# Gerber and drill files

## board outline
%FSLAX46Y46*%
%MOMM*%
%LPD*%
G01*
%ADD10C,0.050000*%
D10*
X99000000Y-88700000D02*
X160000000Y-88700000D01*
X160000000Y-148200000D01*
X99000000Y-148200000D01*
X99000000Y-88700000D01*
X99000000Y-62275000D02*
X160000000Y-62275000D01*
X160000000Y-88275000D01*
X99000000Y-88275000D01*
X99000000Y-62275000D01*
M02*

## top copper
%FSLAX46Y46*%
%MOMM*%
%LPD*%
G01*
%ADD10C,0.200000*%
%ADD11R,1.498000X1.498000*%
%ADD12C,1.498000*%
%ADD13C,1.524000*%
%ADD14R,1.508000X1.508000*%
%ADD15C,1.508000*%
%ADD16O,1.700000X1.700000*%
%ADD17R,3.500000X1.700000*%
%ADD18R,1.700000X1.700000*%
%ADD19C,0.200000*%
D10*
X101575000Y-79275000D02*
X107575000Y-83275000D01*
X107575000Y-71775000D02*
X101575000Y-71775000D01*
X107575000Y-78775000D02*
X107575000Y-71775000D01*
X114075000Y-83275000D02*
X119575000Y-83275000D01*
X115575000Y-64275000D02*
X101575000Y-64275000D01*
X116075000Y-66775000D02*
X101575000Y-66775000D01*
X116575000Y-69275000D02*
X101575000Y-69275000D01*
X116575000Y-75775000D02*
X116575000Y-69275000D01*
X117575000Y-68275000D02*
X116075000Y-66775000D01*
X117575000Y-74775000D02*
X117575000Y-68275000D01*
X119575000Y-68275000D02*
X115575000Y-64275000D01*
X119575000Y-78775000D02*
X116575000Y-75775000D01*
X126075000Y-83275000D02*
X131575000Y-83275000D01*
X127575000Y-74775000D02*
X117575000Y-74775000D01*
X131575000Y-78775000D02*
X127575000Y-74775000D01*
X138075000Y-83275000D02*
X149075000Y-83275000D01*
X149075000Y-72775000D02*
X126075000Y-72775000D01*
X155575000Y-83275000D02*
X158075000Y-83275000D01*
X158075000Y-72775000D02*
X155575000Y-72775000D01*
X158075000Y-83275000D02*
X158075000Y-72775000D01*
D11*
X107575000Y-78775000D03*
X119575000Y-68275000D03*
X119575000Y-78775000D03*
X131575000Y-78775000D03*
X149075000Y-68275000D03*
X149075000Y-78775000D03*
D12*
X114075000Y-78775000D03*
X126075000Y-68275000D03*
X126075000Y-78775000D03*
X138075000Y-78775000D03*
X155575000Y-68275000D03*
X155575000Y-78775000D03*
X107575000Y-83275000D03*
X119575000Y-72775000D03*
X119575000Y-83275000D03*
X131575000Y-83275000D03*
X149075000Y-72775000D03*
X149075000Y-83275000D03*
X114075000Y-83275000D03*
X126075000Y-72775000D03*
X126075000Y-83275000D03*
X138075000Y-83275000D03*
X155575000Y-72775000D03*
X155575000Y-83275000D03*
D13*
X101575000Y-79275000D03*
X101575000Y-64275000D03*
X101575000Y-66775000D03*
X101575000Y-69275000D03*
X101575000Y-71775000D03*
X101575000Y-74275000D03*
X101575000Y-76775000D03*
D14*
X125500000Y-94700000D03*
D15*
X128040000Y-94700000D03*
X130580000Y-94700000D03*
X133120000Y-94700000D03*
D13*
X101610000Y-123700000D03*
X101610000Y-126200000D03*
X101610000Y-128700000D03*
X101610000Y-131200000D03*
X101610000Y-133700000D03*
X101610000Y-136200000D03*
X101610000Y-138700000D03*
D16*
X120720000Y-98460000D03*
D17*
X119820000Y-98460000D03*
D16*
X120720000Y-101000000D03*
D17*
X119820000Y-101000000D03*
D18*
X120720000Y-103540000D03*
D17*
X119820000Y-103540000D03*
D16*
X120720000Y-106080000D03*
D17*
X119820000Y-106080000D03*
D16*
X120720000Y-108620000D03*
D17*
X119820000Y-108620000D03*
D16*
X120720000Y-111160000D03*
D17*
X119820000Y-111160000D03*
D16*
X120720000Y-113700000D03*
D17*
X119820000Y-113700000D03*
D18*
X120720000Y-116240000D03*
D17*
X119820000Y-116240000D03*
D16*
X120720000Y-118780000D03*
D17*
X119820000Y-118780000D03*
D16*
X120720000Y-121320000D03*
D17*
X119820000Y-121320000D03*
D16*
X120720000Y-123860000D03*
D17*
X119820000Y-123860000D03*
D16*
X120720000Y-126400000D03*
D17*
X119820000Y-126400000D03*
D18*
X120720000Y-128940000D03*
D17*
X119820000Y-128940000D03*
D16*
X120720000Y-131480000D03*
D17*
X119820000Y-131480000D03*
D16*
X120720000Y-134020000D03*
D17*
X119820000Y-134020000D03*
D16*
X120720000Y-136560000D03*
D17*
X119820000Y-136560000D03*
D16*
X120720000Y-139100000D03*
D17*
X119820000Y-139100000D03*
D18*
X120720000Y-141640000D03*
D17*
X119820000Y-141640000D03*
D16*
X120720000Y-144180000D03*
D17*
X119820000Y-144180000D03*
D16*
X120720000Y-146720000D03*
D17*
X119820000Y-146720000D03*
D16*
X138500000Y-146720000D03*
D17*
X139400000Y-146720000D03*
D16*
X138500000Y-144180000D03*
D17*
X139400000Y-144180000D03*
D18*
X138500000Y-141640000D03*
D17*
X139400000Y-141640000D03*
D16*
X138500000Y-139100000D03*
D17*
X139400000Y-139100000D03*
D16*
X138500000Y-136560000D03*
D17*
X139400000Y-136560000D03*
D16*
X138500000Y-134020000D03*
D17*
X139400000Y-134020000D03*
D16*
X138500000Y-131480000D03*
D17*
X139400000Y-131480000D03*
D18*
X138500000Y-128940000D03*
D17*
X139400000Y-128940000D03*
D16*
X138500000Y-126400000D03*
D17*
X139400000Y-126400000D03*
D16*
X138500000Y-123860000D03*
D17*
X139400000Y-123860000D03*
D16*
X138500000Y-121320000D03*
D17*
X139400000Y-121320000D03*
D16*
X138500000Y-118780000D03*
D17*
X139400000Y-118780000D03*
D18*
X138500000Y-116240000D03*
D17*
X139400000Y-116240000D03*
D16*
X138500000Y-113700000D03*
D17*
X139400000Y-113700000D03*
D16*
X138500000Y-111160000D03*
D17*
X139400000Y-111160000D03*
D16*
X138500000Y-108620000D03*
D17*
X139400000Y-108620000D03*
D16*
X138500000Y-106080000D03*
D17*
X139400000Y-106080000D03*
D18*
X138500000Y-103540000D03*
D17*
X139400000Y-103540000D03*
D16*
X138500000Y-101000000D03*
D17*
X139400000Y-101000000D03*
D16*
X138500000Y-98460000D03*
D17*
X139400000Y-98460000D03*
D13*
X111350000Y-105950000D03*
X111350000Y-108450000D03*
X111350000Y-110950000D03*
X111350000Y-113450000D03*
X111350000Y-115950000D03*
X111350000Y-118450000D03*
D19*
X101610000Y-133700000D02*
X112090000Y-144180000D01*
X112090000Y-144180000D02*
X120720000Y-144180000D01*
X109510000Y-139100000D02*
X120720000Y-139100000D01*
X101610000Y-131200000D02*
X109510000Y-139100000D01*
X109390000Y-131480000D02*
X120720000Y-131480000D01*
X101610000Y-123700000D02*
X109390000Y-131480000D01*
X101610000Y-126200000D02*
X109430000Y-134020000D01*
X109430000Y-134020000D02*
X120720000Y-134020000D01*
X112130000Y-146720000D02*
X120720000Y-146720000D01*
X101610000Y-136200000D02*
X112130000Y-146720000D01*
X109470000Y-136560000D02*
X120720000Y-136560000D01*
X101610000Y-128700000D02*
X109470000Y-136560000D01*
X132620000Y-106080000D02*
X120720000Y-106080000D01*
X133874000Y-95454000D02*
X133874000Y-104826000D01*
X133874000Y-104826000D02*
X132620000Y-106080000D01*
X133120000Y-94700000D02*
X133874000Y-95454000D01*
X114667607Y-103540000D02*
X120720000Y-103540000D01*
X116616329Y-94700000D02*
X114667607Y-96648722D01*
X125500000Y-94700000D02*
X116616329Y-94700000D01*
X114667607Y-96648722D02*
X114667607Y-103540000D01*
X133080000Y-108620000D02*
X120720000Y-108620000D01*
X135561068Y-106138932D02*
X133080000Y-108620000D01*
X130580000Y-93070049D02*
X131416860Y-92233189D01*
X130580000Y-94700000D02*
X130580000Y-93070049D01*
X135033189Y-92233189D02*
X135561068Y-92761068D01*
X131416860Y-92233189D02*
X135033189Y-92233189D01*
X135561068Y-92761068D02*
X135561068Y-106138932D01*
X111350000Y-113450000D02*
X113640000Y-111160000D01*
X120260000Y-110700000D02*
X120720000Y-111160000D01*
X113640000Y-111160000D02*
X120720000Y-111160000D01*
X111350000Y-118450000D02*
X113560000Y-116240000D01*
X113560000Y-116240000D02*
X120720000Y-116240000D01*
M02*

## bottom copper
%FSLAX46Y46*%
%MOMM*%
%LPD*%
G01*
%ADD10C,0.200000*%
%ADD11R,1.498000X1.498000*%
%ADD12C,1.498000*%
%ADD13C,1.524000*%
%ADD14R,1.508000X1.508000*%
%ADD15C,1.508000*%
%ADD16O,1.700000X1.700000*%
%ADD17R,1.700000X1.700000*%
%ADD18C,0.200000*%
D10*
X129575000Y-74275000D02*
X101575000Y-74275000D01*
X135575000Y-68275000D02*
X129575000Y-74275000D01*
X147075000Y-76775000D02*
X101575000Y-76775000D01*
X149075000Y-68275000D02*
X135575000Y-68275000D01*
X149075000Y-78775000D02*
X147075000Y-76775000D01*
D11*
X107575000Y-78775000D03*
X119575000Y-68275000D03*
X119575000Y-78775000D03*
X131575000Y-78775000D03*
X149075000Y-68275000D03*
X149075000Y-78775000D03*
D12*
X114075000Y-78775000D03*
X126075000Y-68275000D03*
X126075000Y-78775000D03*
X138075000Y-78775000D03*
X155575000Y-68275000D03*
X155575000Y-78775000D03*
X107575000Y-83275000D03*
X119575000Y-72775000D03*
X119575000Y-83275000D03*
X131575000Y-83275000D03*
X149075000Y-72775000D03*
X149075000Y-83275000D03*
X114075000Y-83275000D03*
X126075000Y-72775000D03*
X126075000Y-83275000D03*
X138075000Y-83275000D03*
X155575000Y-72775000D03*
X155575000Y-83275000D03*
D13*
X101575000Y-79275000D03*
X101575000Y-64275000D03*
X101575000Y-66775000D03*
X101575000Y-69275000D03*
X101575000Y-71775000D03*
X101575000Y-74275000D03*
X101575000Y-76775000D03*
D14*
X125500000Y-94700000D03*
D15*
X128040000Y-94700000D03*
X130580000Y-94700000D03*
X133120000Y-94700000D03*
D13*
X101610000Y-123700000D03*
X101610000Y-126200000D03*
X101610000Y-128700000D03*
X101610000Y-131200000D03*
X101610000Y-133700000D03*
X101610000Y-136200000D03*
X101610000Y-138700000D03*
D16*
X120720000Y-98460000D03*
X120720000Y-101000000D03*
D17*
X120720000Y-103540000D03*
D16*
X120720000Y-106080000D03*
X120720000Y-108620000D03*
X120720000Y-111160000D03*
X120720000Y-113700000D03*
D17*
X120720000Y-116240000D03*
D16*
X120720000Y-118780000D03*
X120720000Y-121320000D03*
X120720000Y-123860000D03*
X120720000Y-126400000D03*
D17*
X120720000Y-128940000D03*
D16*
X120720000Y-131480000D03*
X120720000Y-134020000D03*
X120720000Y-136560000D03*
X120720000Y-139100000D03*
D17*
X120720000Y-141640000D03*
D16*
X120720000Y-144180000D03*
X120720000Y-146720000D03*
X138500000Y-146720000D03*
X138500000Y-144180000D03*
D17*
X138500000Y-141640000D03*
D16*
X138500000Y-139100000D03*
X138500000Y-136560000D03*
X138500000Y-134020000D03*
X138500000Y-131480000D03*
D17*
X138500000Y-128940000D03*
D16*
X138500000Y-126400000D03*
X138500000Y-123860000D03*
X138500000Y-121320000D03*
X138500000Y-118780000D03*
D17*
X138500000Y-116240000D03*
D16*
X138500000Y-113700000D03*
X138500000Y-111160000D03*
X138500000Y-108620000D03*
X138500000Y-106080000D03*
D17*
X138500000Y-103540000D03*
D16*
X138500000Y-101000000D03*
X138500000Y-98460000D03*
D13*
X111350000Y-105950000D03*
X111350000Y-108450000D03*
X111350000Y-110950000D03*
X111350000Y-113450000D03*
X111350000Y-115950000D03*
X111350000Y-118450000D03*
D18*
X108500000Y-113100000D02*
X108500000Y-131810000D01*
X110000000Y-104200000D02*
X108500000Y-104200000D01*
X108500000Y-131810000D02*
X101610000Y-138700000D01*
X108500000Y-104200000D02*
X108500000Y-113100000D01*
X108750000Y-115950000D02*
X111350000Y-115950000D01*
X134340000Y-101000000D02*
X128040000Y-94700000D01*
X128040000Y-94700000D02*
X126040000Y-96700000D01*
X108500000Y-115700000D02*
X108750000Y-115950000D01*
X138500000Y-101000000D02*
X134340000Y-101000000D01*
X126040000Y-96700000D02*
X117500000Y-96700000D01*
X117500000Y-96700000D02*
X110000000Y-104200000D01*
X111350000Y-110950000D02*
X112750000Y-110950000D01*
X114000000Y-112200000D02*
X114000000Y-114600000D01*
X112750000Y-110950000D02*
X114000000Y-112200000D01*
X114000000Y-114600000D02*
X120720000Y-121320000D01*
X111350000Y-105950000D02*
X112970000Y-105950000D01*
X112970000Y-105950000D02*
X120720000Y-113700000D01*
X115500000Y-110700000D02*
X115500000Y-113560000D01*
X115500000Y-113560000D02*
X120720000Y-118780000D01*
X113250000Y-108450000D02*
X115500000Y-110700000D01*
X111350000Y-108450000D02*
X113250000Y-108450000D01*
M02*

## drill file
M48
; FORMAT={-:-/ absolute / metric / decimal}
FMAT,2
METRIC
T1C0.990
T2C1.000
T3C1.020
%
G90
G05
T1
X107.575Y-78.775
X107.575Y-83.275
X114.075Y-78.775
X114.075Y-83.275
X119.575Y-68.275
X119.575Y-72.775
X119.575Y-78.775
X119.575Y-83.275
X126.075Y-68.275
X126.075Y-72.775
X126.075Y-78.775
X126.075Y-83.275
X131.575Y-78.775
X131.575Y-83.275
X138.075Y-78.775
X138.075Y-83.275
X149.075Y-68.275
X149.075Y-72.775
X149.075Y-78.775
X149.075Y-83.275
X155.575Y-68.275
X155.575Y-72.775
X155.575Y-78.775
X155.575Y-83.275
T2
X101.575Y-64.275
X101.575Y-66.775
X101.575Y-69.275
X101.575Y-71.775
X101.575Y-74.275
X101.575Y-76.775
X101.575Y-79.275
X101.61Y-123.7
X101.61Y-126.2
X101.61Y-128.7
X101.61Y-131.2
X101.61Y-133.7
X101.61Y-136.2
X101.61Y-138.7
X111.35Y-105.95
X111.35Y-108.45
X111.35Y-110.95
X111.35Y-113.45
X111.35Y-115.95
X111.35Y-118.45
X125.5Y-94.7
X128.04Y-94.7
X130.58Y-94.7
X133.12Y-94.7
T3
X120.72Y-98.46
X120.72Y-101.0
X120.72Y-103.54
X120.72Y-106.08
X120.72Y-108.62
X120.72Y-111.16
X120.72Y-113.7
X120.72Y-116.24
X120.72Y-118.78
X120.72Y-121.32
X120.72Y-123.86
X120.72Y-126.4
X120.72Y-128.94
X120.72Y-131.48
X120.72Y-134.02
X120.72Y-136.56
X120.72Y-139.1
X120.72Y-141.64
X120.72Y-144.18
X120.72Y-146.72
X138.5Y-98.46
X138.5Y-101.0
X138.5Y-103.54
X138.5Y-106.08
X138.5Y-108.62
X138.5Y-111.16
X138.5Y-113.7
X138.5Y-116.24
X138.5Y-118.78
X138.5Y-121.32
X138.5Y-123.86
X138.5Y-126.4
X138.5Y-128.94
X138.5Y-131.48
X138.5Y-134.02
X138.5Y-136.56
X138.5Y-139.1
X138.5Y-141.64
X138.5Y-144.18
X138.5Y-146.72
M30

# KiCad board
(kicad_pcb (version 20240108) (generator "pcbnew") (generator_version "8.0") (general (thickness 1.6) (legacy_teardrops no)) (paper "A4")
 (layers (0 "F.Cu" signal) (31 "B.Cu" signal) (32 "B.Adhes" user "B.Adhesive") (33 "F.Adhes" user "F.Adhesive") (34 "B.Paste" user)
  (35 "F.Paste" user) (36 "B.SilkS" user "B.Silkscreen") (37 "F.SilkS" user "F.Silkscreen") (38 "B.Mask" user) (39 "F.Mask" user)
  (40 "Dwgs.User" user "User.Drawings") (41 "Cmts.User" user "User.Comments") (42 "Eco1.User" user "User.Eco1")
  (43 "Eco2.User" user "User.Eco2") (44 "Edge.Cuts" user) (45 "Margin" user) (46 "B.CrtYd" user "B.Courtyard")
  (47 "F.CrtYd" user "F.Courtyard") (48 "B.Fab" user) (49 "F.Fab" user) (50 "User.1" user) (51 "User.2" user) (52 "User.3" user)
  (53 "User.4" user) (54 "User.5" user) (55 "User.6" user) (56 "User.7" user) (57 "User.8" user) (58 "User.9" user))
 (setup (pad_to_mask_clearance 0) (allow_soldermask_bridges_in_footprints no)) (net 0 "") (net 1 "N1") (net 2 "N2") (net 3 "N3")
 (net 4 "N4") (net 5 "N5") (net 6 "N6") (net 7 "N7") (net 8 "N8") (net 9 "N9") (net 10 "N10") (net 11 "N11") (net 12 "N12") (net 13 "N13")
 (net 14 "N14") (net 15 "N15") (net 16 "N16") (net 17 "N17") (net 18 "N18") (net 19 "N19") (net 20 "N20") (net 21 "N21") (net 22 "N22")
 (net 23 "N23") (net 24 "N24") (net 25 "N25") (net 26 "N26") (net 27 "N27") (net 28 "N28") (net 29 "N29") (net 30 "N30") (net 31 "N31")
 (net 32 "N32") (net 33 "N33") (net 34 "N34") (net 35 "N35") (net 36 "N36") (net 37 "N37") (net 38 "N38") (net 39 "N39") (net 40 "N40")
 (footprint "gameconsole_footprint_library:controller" (layer "F.Cu") (at 99.575 62.775)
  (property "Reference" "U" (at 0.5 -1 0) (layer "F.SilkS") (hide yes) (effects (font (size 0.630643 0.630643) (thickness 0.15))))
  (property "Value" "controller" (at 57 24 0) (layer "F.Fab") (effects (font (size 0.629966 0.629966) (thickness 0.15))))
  (fp_line (start 2 16.5) (end 8 20.5) (stroke (width 0.2) (type default)) (layer "F.Cu"))
  (fp_line (start 8 9) (end 2 9) (stroke (width 0.2) (type default)) (layer "F.Cu"))
  (fp_line (start 8 16) (end 8 9) (stroke (width 0.2) (type default)) (layer "F.Cu"))
  (fp_line (start 14.5 20.5) (end 20 20.5) (stroke (width 0.2) (type default)) (layer "F.Cu"))
  (fp_line (start 16 1.5) (end 2 1.5) (stroke (width 0.2) (type default)) (layer "F.Cu"))
  (fp_line (start 16.5 4) (end 2 4) (stroke (width 0.2) (type default)) (layer "F.Cu"))
  (fp_line (start 17 6.5) (end 2 6.5) (stroke (width 0.2) (type default)) (layer "F.Cu"))
  (fp_line (start 17 13) (end 17 6.5) (stroke (width 0.2) (type default)) (layer "F.Cu"))
  (fp_line (start 18 5.5) (end 16.5 4) (stroke (width 0.2) (type default)) (layer "F.Cu"))
  (fp_line (start 18 12) (end 18 5.5) (stroke (width 0.2) (type default)) (layer "F.Cu"))
  (fp_line (start 20 5.5) (end 16 1.5) (stroke (width 0.2) (type default)) (layer "F.Cu"))
  (fp_line (start 20 16) (end 17 13) (stroke (width 0.2) (type default)) (layer "F.Cu"))
  (fp_line (start 26.5 20.5) (end 32 20.5) (stroke (width 0.2) (type default)) (layer "F.Cu"))
  (fp_line (start 28 12) (end 18 12) (stroke (width 0.2) (type default)) (layer "F.Cu"))
  (fp_line (start 32 16) (end 28 12) (stroke (width 0.2) (type default)) (layer "F.Cu"))
  (fp_line (start 38.5 20.5) (end 49.5 20.5) (stroke (width 0.2) (type default)) (layer "F.Cu"))
  (fp_line (start 49.5 10) (end 26.5 10) (stroke (width 0.2) (type default)) (layer "F.Cu"))
  (fp_line (start 56 20.5) (end 58.5 20.5) (stroke (width 0.2) (type default)) (layer "F.Cu"))
  (fp_line (start 58.5 10) (end 56 10) (stroke (width 0.2) (type default)) (layer "F.Cu"))
  (fp_line (start 58.5 20.5) (end 58.5 10) (stroke (width 0.2) (type default)) (layer "F.Cu"))
  (fp_line (start 30 11.5) (end 2 11.5) (stroke (width 0.2) (type default)) (layer "B.Cu"))
  (fp_line (start 36 5.5) (end 30 11.5) (stroke (width 0.2) (type default)) (layer "B.Cu"))
  (fp_line (start 47.5 14) (end 2 14) (stroke (width 0.2) (type default)) (layer "B.Cu"))
  (fp_line (start 49.5 5.5) (end 36 5.5) (stroke (width 0.2) (type default)) (layer "B.Cu"))
  (fp_line (start 49.5 16) (end 47.5 14) (stroke (width 0.2) (type default)) (layer "B.Cu"))
  (pad "1" thru_hole rect (at 8 16) (size 1.498 1.498) (drill 0.99) (layers "*.Cu" "*.Mask") (remove_unused_layers no)
   (solder_mask_margin 0.102))
  (pad "1" thru_hole rect (at 20 5.5) (size 1.498 1.498) (drill 0.99) (layers "*.Cu" "*.Mask") (remove_unused_layers no)
   (solder_mask_margin 0.102))
  (pad "1" thru_hole rect (at 20 16) (size 1.498 1.498) (drill 0.99) (layers "*.Cu" "*.Mask") (remove_unused_layers no)
   (solder_mask_margin 0.102))
  (pad "1" thru_hole rect (at 32 16) (size 1.498 1.498) (drill 0.99) (layers "*.Cu" "*.Mask") (remove_unused_layers no)
   (solder_mask_margin 0.102))
  (pad "1" thru_hole rect (at 49.5 5.5) (size 1.498 1.498) (drill 0.99) (layers "*.Cu" "*.Mask") (remove_unused_layers no)
   (solder_mask_margin 0.102))
  (pad "1" thru_hole rect (at 49.5 16) (size 1.498 1.498) (drill 0.99) (layers "*.Cu" "*.Mask") (remove_unused_layers no)
   (solder_mask_margin 0.102))
  (pad "2" thru_hole circle (at 14.5 16) (size 1.498 1.498) (drill 0.99) (layers "*.Cu" "*.Mask") (remove_unused_layers no)
   (solder_mask_margin 0.102))
  (pad "2" thru_hole circle (at 26.5 5.5) (size 1.498 1.498) (drill 0.99) (layers "*.Cu" "*.Mask") (remove_unused_layers no)
   (solder_mask_margin 0.102))
  (pad "2" thru_hole circle (at 26.5 16) (size 1.498 1.498) (drill 0.99) (layers "*.Cu" "*.Mask") (remove_unused_layers no)
   (solder_mask_margin 0.102))
  (pad "2" thru_hole circle (at 38.5 16) (size 1.498 1.498) (drill 0.99) (layers "*.Cu" "*.Mask") (remove_unused_layers no)
   (solder_mask_margin 0.102))
  (pad "2" thru_hole circle (at 56 5.5) (size 1.498 1.498) (drill 0.99) (layers "*.Cu" "*.Mask") (remove_unused_layers no)
   (solder_mask_margin 0.102))
  (pad "2" thru_hole circle (at 56 16) (size 1.498 1.498) (drill 0.99) (layers "*.Cu" "*.Mask") (remove_unused_layers no)
   (solder_mask_margin 0.102))
  (pad "3" thru_hole circle (at 8 20.5) (size 1.498 1.498) (drill 0.99) (layers "*.Cu" "*.Mask") (remove_unused_layers no)
   (solder_mask_margin 0.102))
  (pad "3" thru_hole circle (at 20 10) (size 1.498 1.498) (drill 0.99) (layers "*.Cu" "*.Mask") (remove_unused_layers no)
   (solder_mask_margin 0.102))
  (pad "3" thru_hole circle (at 20 20.5) (size 1.498 1.498) (drill 0.99) (layers "*.Cu" "*.Mask") (remove_unused_layers no)
   (solder_mask_margin 0.102))
  (pad "3" thru_hole circle (at 32 20.5) (size 1.498 1.498) (drill 0.99) (layers "*.Cu" "*.Mask") (remove_unused_layers no)
   (solder_mask_margin 0.102))
  (pad "3" thru_hole circle (at 49.5 10) (size 1.498 1.498) (drill 0.99) (layers "*.Cu" "*.Mask") (remove_unused_layers no)
   (solder_mask_margin 0.102))
  (pad "3" thru_hole circle (at 49.5 20.5) (size 1.498 1.498) (drill 0.99) (layers "*.Cu" "*.Mask") (remove_unused_layers no)
   (solder_mask_margin 0.102))
  (pad "4" thru_hole circle (at 14.5 20.5) (size 1.498 1.498) (drill 0.99) (layers "*.Cu" "*.Mask") (remove_unused_layers no)
   (solder_mask_margin 0.102))
  (pad "4" thru_hole circle (at 26.5 10) (size 1.498 1.498) (drill 0.99) (layers "*.Cu" "*.Mask") (remove_unused_layers no)
   (solder_mask_margin 0.102))
  (pad "4" thru_hole circle (at 26.5 20.5) (size 1.498 1.498) (drill 0.99) (layers "*.Cu" "*.Mask") (remove_unused_layers no)
   (solder_mask_margin 0.102))
  (pad "4" thru_hole circle (at 38.5 20.5) (size 1.498 1.498) (drill 0.99) (layers "*.Cu" "*.Mask") (remove_unused_layers no)
   (solder_mask_margin 0.102))
  (pad "4" thru_hole circle (at 56 10) (size 1.498 1.498) (drill 0.99) (layers "*.Cu" "*.Mask") (remove_unused_layers no)
   (solder_mask_margin 0.102))
  (pad "4" thru_hole circle (at 56 20.5) (size 1.498 1.498) (drill 0.99) (layers "*.Cu" "*.Mask") (remove_unused_layers no)
   (solder_mask_margin 0.102))
  (pad "5" thru_hole circle (at 2 16.5) (size 1.524 1.524) (drill 1) (layers "*.Cu" "*.Mask") (remove_unused_layers no))
  (pad "6" thru_hole circle (at 2 1.5) (size 1.524 1.524) (drill 1) (layers "*.Cu" "*.Mask") (remove_unused_layers no))
  (pad "7" thru_hole circle (at 2 4) (size 1.524 1.524) (drill 1) (layers "*.Cu" "*.Mask") (remove_unused_layers no))
  (pad "8" thru_hole circle (at 2 6.5) (size 1.524 1.524) (drill 1) (layers "*.Cu" "*.Mask") (remove_unused_layers no))
  (pad "9" thru_hole circle (at 2 9) (size 1.524 1.524) (drill 1) (layers "*.Cu" "*.Mask") (remove_unused_layers no))
  (pad "10" thru_hole circle (at 2 11.5) (size 1.524 1.524) (drill 1) (layers "*.Cu" "*.Mask") (remove_unused_layers no))
  (pad "11" thru_hole circle (at 2 14) (size 1.524 1.524) (drill 1) (layers "*.Cu" "*.Mask") (remove_unused_layers no)))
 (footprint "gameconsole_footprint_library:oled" (layer "F.Cu") (at 129.31 106.2)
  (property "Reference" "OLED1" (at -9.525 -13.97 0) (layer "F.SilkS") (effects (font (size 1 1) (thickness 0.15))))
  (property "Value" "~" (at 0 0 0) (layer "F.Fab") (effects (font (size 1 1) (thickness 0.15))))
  (pad "1" thru_hole rect (at -3.81 -11.5) (size 1.508 1.508) (drill 1) (layers "*.Cu" "*.Mask") (remove_unused_layers no) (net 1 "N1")
   (solder_mask_margin 0.102))
  (pad "2" thru_hole circle (at -1.27 -11.5) (size 1.508 1.508) (drill 1) (layers "*.Cu" "*.Mask") (remove_unused_layers no) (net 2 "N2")
   (solder_mask_margin 0.102))
  (pad "3" thru_hole circle (at 1.27 -11.5) (size 1.508 1.508) (drill 1) (layers "*.Cu" "*.Mask") (remove_unused_layers no) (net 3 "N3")
   (solder_mask_margin 0.102))
  (pad "4" thru_hole circle (at 3.81 -11.5) (size 1.508 1.508) (drill 1) (layers "*.Cu" "*.Mask") (remove_unused_layers no) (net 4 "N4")
   (solder_mask_margin 0.102)))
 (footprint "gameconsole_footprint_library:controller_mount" (layer "F.Cu") (at 129.61 134.2)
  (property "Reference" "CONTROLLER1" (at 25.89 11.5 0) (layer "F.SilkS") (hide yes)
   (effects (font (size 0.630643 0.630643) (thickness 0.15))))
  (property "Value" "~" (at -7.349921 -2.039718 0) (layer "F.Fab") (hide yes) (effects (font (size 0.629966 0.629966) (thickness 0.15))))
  (pad "1" thru_hole circle (at -28 -10.5) (size 1.524 1.524) (drill 1) (layers "*.Cu" "*.Mask") (remove_unused_layers no) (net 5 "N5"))
  (pad "2" thru_hole circle (at -28 -8) (size 1.524 1.524) (drill 1) (layers "*.Cu" "*.Mask") (remove_unused_layers no) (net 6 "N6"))
  (pad "3" thru_hole circle (at -28 -5.5) (size 1.524 1.524) (drill 1) (layers "*.Cu" "*.Mask") (remove_unused_layers no) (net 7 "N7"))
  (pad "4" thru_hole circle (at -28 -3) (size 1.524 1.524) (drill 1) (layers "*.Cu" "*.Mask") (remove_unused_layers no) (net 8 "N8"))
  (pad "5" thru_hole circle (at -28 -0.5) (size 1.524 1.524) (drill 1) (layers "*.Cu" "*.Mask") (remove_unused_layers no) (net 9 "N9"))
  (pad "6" thru_hole circle (at -28 2) (size 1.524 1.524) (drill 1) (layers "*.Cu" "*.Mask") (remove_unused_layers no) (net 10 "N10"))
  (pad "7" thru_hole circle (at -28 4.5) (size 1.524 1.524) (drill 1) (layers "*.Cu" "*.Mask") (remove_unused_layers no) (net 2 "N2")))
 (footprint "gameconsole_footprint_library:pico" (layer "F.Cu") (at 129.61 122.59)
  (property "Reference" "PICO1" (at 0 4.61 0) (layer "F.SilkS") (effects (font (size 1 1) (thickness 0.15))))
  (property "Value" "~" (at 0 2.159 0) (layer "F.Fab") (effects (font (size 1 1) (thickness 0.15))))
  (pad "1" thru_hole oval (at -8.89 -24.13) (size 1.7 1.7) (drill 1.02) (layers "*.Cu" "*.Mask") (remove_unused_layers no) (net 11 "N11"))
  (pad "1" smd rect (at -8.89 -24.13) (size 3.5 1.7) (drill (offset -0.9 0)) (layers "F.Cu" "F.Mask") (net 11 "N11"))
  (pad "2" thru_hole oval (at -8.89 -21.59) (size 1.7 1.7) (drill 1.02) (layers "*.Cu" "*.Mask") (remove_unused_layers no) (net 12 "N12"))
  (pad "2" smd rect (at -8.89 -21.59) (size 3.5 1.7) (drill (offset -0.9 0)) (layers "F.Cu" "F.Mask") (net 12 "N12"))
  (pad "3" thru_hole rect (at -8.89 -19.05) (size 1.7 1.7) (drill 1.02) (layers "*.Cu" "*.Mask") (remove_unused_layers no) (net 1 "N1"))
  (pad "3" smd rect (at -8.89 -19.05) (size 3.5 1.7) (drill (offset -0.9 0)) (layers "F.Cu" "F.Mask") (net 1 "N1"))
  (pad "4" thru_hole oval (at -8.89 -16.51) (size 1.7 1.7) (drill 1.02) (layers "*.Cu" "*.Mask") (remove_unused_layers no) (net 4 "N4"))
  (pad "4" smd rect (at -8.89 -16.51) (size 3.5 1.7) (drill (offset -0.9 0)) (layers "F.Cu" "F.Mask") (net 4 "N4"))
  (pad "5" thru_hole oval (at -8.89 -13.97) (size 1.7 1.7) (drill 1.02) (layers "*.Cu" "*.Mask") (remove_unused_layers no) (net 3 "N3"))
  (pad "5" smd rect (at -8.89 -13.97) (size 3.5 1.7) (drill (offset -0.9 0)) (layers "F.Cu" "F.Mask") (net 3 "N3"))
  (pad "6" thru_hole oval (at -8.89 -11.43) (size 1.7 1.7) (drill 1.02) (layers "*.Cu" "*.Mask") (remove_unused_layers no) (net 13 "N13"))
  (pad "6" smd rect (at -8.89 -11.43) (size 3.5 1.7) (drill (offset -0.9 0)) (layers "F.Cu" "F.Mask") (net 13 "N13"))
  (pad "7" thru_hole oval (at -8.89 -8.89) (size 1.7 1.7) (drill 1.02) (layers "*.Cu" "*.Mask") (remove_unused_layers no) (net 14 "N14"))
  (pad "7" smd rect (at -8.89 -8.89) (size 3.5 1.7) (drill (offset -0.9 0)) (layers "F.Cu" "F.Mask") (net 14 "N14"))
  (pad "8" thru_hole rect (at -8.89 -6.35) (size 1.7 1.7) (drill 1.02) (layers "*.Cu" "*.Mask") (remove_unused_layers no) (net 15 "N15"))
  (pad "8" smd rect (at -8.89 -6.35) (size 3.5 1.7) (drill (offset -0.9 0)) (layers "F.Cu" "F.Mask") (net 15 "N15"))
  (pad "9" thru_hole oval (at -8.89 -3.81) (size 1.7 1.7) (drill 1.02) (layers "*.Cu" "*.Mask") (remove_unused_layers no) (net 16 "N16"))
  (pad "9" smd rect (at -8.89 -3.81) (size 3.5 1.7) (drill (offset -0.9 0)) (layers "F.Cu" "F.Mask") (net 16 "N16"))
  (pad "10" thru_hole oval (at -8.89 -1.27) (size 1.7 1.7) (drill 1.02) (layers "*.Cu" "*.Mask") (remove_unused_layers no) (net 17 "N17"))
  (pad "10" smd rect (at -8.89 -1.27) (size 3.5 1.7) (drill (offset -0.9 0)) (layers "F.Cu" "F.Mask") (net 17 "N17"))
  (pad "11" thru_hole oval (at -8.89 1.27) (size 1.7 1.7) (drill 1.02) (layers "*.Cu" "*.Mask") (remove_unused_layers no) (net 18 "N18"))
  (pad "11" smd rect (at -8.89 1.27) (size 3.5 1.7) (drill (offset -0.9 0)) (layers "F.Cu" "F.Mask") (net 18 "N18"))
  (pad "12" thru_hole oval (at -8.89 3.81) (size 1.7 1.7) (drill 1.02) (layers "*.Cu" "*.Mask") (remove_unused_layers no) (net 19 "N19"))
  (pad "12" smd rect (at -8.89 3.81) (size 3.5 1.7) (drill (offset -0.9 0)) (layers "F.Cu" "F.Mask") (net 19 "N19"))
  (pad "13" thru_hole rect (at -8.89 6.35) (size 1.7 1.7) (drill 1.02) (layers "*.Cu" "*.Mask") (remove_unused_layers no) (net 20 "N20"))
  (pad "13" smd rect (at -8.89 6.35) (size 3.5 1.7) (drill (offset -0.9 0)) (layers "F.Cu" "F.Mask") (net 20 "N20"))
  (pad "14" thru_hole oval (at -8.89 8.89) (size 1.7 1.7) (drill 1.02) (layers "*.Cu" "*.Mask") (remove_unused_layers no) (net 5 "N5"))
  (pad "14" smd rect (at -8.89 8.89) (size 3.5 1.7) (drill (offset -0.9 0)) (layers "F.Cu" "F.Mask") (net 5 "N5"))
  (pad "15" thru_hole oval (at -8.89 11.43) (size 1.7 1.7) (drill 1.02) (layers "*.Cu" "*.Mask") (remove_unused_layers no) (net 6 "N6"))
  (pad "15" smd rect (at -8.89 11.43) (size 3.5 1.7) (drill (offset -0.9 0)) (layers "F.Cu" "F.Mask") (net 6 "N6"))
  (pad "16" thru_hole oval (at -8.89 13.97) (size 1.7 1.7) (drill 1.02) (layers "*.Cu" "*.Mask") (remove_unused_layers no) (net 7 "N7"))
  (pad "16" smd rect (at -8.89 13.97) (size 3.5 1.7) (drill (offset -0.9 0)) (layers "F.Cu" "F.Mask") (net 7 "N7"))
  (pad "17" thru_hole oval (at -8.89 16.51) (size 1.7 1.7) (drill 1.02) (layers "*.Cu" "*.Mask") (remove_unused_layers no) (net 8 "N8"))
  (pad "17" smd rect (at -8.89 16.51) (size 3.5 1.7) (drill (offset -0.9 0)) (layers "F.Cu" "F.Mask") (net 8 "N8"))
  (pad "18" thru_hole rect (at -8.89 19.05) (size 1.7 1.7) (drill 1.02) (layers "*.Cu" "*.Mask") (remove_unused_layers no) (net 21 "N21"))
  (pad "18" smd rect (at -8.89 19.05) (size 3.5 1.7) (drill (offset -0.9 0)) (layers "F.Cu" "F.Mask") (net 21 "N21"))
  (pad "19" thru_hole oval (at -8.89 21.59) (size 1.7 1.7) (drill 1.02) (layers "*.Cu" "*.Mask") (remove_unused_layers no) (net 9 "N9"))
  (pad "19" smd rect (at -8.89 21.59) (size 3.5 1.7) (drill (offset -0.9 0)) (layers "F.Cu" "F.Mask") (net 9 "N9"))
  (pad "20" thru_hole oval (at -8.89 24.13) (size 1.7 1.7) (drill 1.02) (layers "*.Cu" "*.Mask") (remove_unused_layers no) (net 10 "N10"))
  (pad "20" smd rect (at -8.89 24.13) (size 3.5 1.7) (drill (offset -0.9 0)) (layers "F.Cu" "F.Mask") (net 10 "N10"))
  (pad "21" thru_hole oval (at 8.89 24.13) (size 1.7 1.7) (drill 1.02) (layers "*.Cu" "*.Mask") (remove_unused_layers no) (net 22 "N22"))
  (pad "21" smd rect (at 8.89 24.13) (size 3.5 1.7) (drill (offset 0.9 0)) (layers "F.Cu" "F.Mask") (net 22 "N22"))
  (pad "22" thru_hole oval (at 8.89 21.59) (size 1.7 1.7) (drill 1.02) (layers "*.Cu" "*.Mask") (remove_unused_layers no) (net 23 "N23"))
  (pad "22" smd rect (at 8.89 21.59) (size 3.5 1.7) (drill (offset 0.9 0)) (layers "F.Cu" "F.Mask") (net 23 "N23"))
  (pad "23" thru_hole rect (at 8.89 19.05) (size 1.7 1.7) (drill 1.02) (layers "*.Cu" "*.Mask") (remove_unused_layers no) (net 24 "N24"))
  (pad "23" smd rect (at 8.89 19.05) (size 3.5 1.7) (drill (offset 0.9 0)) (layers "F.Cu" "F.Mask") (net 24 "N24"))
  (pad "24" thru_hole oval (at 8.89 16.51) (size 1.7 1.7) (drill 1.02) (layers "*.Cu" "*.Mask") (remove_unused_layers no) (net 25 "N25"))
  (pad "24" smd rect (at 8.89 16.51) (size 3.5 1.7) (drill (offset 0.9 0)) (layers "F.Cu" "F.Mask") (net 25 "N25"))
  (pad "25" thru_hole oval (at 8.89 13.97) (size 1.7 1.7) (drill 1.02) (layers "*.Cu" "*.Mask") (remove_unused_layers no) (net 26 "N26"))
  (pad "25" smd rect (at 8.89 13.97) (size 3.5 1.7) (drill (offset 0.9 0)) (layers "F.Cu" "F.Mask") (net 26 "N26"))
  (pad "26" thru_hole oval (at 8.89 11.43) (size 1.7 1.7) (drill 1.02) (layers "*.Cu" "*.Mask") (remove_unused_layers no) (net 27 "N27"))
  (pad "26" smd rect (at 8.89 11.43) (size 3.5 1.7) (drill (offset 0.9 0)) (layers "F.Cu" "F.Mask") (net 27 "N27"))
  (pad "27" thru_hole oval (at 8.89 8.89) (size 1.7 1.7) (drill 1.02) (layers "*.Cu" "*.Mask") (remove_unused_layers no) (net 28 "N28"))
  (pad "27" smd rect (at 8.89 8.89) (size 3.5 1.7) (drill (offset 0.9 0)) (layers "F.Cu" "F.Mask") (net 28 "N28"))
  (pad "28" thru_hole rect (at 8.89 6.35) (size 1.7 1.7) (drill 1.02) (layers "*.Cu" "*.Mask") (remove_unused_layers no) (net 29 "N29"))
  (pad "28" smd rect (at 8.89 6.35) (size 3.5 1.7) (drill (offset 0.9 0)) (layers "F.Cu" "F.Mask") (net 29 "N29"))
  (pad "29" thru_hole oval (at 8.89 3.81) (size 1.7 1.7) (drill 1.02) (layers "*.Cu" "*.Mask") (remove_unused_layers no) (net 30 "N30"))
  (pad "29" smd rect (at 8.89 3.81) (size 3.5 1.7) (drill (offset 0.9 0)) (layers "F.Cu" "F.Mask") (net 30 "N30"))
  (pad "30" thru_hole oval (at 8.89 1.27) (size 1.7 1.7) (drill 1.02) (layers "*.Cu" "*.Mask") (remove_unused_layers no) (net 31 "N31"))
  (pad "30" smd rect (at 8.89 1.27) (size 3.5 1.7) (drill (offset 0.9 0)) (layers "F.Cu" "F.Mask") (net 31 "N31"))
  (pad "31" thru_hole oval (at 8.89 -1.27) (size 1.7 1.7) (drill 1.02) (layers "*.Cu" "*.Mask") (remove_unused_layers no) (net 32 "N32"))
  (pad "31" smd rect (at 8.89 -1.27) (size 3.5 1.7) (drill (offset 0.9 0)) (layers "F.Cu" "F.Mask") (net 32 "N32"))
  (pad "32" thru_hole oval (at 8.89 -3.81) (size 1.7 1.7) (drill 1.02) (layers "*.Cu" "*.Mask") (remove_unused_layers no) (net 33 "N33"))
  (pad "32" smd rect (at 8.89 -3.81) (size 3.5 1.7) (drill (offset 0.9 0)) (layers "F.Cu" "F.Mask") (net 33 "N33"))
  (pad "33" thru_hole rect (at 8.89 -6.35) (size 1.7 1.7) (drill 1.02) (layers "*.Cu" "*.Mask") (remove_unused_layers no) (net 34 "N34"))
  (pad "33" smd rect (at 8.89 -6.35) (size 3.5 1.7) (drill (offset 0.9 0)) (layers "F.Cu" "F.Mask") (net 34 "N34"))
  (pad "34" thru_hole oval (at 8.89 -8.89) (size 1.7 1.7) (drill 1.02) (layers "*.Cu" "*.Mask") (remove_unused_layers no) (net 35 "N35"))
  (pad "34" smd rect (at 8.89 -8.89) (size 3.5 1.7) (drill (offset 0.9 0)) (layers "F.Cu" "F.Mask") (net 35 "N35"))
  (pad "35" thru_hole oval (at 8.89 -11.43) (size 1.7 1.7) (drill 1.02) (layers "*.Cu" "*.Mask") (remove_unused_layers no) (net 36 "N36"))
  (pad "35" smd rect (at 8.89 -11.43) (size 3.5 1.7) (drill (offset 0.9 0)) (layers "F.Cu" "F.Mask") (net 36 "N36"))
  (pad "36" thru_hole oval (at 8.89 -13.97) (size 1.7 1.7) (drill 1.02) (layers "*.Cu" "*.Mask") (remove_unused_layers no) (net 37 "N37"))
  (pad "36" smd rect (at 8.89 -13.97) (size 3.5 1.7) (drill (offset 0.9 0)) (layers "F.Cu" "F.Mask") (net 37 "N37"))
  (pad "37" thru_hole oval (at 8.89 -16.51) (size 1.7 1.7) (drill 1.02) (layers "*.Cu" "*.Mask") (remove_unused_layers no) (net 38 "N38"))
  (pad "37" smd rect (at 8.89 -16.51) (size 3.5 1.7) (drill (offset 0.9 0)) (layers "F.Cu" "F.Mask") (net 38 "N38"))
  (pad "38" thru_hole rect (at 8.89 -19.05) (size 1.7 1.7) (drill 1.02) (layers "*.Cu" "*.Mask") (remove_unused_layers no) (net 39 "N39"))
  (pad "38" smd rect (at 8.89 -19.05) (size 3.5 1.7) (drill (offset 0.9 0)) (layers "F.Cu" "F.Mask") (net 39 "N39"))
  (pad "39" thru_hole oval (at 8.89 -21.59) (size 1.7 1.7) (drill 1.02) (layers "*.Cu" "*.Mask") (remove_unused_layers no) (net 2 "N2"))
  (pad "39" smd rect (at 8.89 -21.59) (size 3.5 1.7) (drill (offset 0.9 0)) (layers "F.Cu" "F.Mask") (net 2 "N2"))
  (pad "40" thru_hole oval (at 8.89 -24.13) (size 1.7 1.7) (drill 1.02) (layers "*.Cu" "*.Mask") (remove_unused_layers no) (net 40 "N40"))
  (pad "40" smd rect (at 8.89 -24.13) (size 3.5 1.7) (drill (offset 0.9 0)) (layers "F.Cu" "F.Mask") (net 40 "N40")))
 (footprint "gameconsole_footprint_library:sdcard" (layer "B.Cu") (at 108.1 100.2 -90)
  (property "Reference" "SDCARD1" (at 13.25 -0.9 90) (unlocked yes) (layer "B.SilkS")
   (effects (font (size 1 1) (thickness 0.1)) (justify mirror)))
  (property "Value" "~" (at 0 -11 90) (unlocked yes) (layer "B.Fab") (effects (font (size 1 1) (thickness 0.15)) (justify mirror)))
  (pad "1" thru_hole circle (at 5.75 -3.25 270) (size 1.524 1.524) (drill 1) (layers "*.Cu" "*.Mask") (remove_unused_layers no)
   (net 14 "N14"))
  (pad "2" thru_hole circle (at 8.25 -3.25 270) (size 1.524 1.524) (drill 1) (layers "*.Cu" "*.Mask") (remove_unused_layers no)
   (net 16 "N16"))
  (pad "3" thru_hole circle (at 10.75 -3.25 270) (size 1.524 1.524) (drill 1) (layers "*.Cu" "*.Mask") (remove_unused_layers no)
   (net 17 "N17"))
  (pad "4" thru_hole circle (at 13.25 -3.25 270) (size 1.524 1.524) (drill 1) (layers "*.Cu" "*.Mask") (remove_unused_layers no)
   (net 13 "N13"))
  (pad "5" thru_hole circle (at 15.75 -3.25 270) (size 1.524 1.524) (drill 1) (layers "*.Cu" "*.Mask") (remove_unused_layers no)
   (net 2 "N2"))
  (pad "6" thru_hole circle (at 18.25 -3.25 270) (size 1.524 1.524) (drill 1) (layers "*.Cu" "*.Mask") (remove_unused_layers no)
   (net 15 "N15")))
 (gr_rect (start 99 88.7) (end 160 148.2) (stroke (width 0.05) (type default)) (fill none) (layer "Edge.Cuts"))
 (gr_rect (start 99 62.275) (end 160 88.275) (stroke (width 0.05) (type default)) (fill none) (layer "Edge.Cuts"))
 (segment (start 101.61 133.7) (end 112.09 144.18) (width 0.2) (layer "F.Cu") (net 9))
 (segment (start 112.09 144.18) (end 120.72 144.18) (width 0.2) (layer "F.Cu") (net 9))
 (segment (start 109.51 139.1) (end 120.72 139.1) (width 0.2) (layer "F.Cu") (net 8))
 (segment (start 101.61 131.2) (end 109.51 139.1) (width 0.2) (layer "F.Cu") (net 8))
 (segment (start 109.39 131.48) (end 120.72 131.48) (width 0.2) (layer "F.Cu") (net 5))
 (segment (start 101.61 123.7) (end 109.39 131.48) (width 0.2) (layer "F.Cu") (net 5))
 (segment (start 101.61 126.2) (end 109.43 134.02) (width 0.2) (layer "F.Cu") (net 6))
 (segment (start 109.43 134.02) (end 120.72 134.02) (width 0.2) (layer "F.Cu") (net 6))
 (segment (start 108.5 113.1) (end 108.5 131.81) (width 0.2) (layer "B.Cu") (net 2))
 (segment (start 110 104.2) (end 108.5 104.2) (width 0.2) (layer "B.Cu") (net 2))
 (segment (start 108.5 131.81) (end 101.61 138.7) (width 0.2) (layer "B.Cu") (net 2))
 (segment (start 108.5 104.2) (end 108.5 113.1) (width 0.2) (layer "B.Cu") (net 2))
 (segment (start 108.75 115.95) (end 111.35 115.95) (width 0.2) (layer "B.Cu") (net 2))
 (segment (start 134.34 101) (end 128.04 94.7) (width 0.2) (layer "B.Cu") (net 2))
 (segment (start 128.04 94.7) (end 126.04 96.7) (width 0.2) (layer "B.Cu") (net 2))
 (segment (start 108.5 115.7) (end 108.75 115.95) (width 0.2) (layer "B.Cu") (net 2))
 (segment (start 138.5 101) (end 134.34 101) (width 0.2) (layer "B.Cu") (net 2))
 (segment (start 126.04 96.7) (end 117.5 96.7) (width 0.2) (layer "B.Cu") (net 2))
 (segment (start 117.5 96.7) (end 110 104.2) (width 0.2) (layer "B.Cu") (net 2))
 (segment (start 112.13 146.72) (end 120.72 146.72) (width 0.2) (layer "F.Cu") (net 10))
 (segment (start 101.61 136.2) (end 112.13 146.72) (width 0.2) (layer "F.Cu") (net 10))
 (segment (start 109.47 136.56) (end 120.72 136.56) (width 0.2) (layer "F.Cu") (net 7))
 (segment (start 101.61 128.7) (end 109.47 136.56) (width 0.2) (layer "F.Cu") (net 7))
 (segment (start 132.62 106.08) (end 120.72 106.08) (width 0.2) (layer "F.Cu") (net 4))
 (segment (start 133.874 95.454) (end 133.874 104.826) (width 0.2) (layer "F.Cu") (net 4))
 (segment (start 133.874 104.826) (end 132.62 106.08) (width 0.2) (layer "F.Cu") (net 4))
 (segment (start 133.12 94.7) (end 133.874 95.454) (width 0.2) (layer "F.Cu") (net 4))
 (segment (start 114.667607 103.54) (end 120.72 103.54) (width 0.2) (layer "F.Cu") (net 1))
 (segment (start 116.616329 94.7) (end 114.667607 96.648722) (width 0.2) (layer "F.Cu") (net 1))
 (segment (start 125.5 94.7) (end 116.616329 94.7) (width 0.2) (layer "F.Cu") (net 1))
 (segment (start 114.667607 96.648722) (end 114.667607 103.54) (width 0.2) (layer "F.Cu") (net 1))
 (segment (start 133.08 108.62) (end 120.72 108.62) (width 0.2) (layer "F.Cu") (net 3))
 (segment (start 135.561068 106.138932) (end 133.08 108.62) (width 0.2) (layer "F.Cu") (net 3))
 (segment (start 130.58 93.070049) (end 131.41686 92.233189) (width 0.2) (layer "F.Cu") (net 3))
 (segment (start 130.58 94.7) (end 130.58 93.070049) (width 0.2) (layer "F.Cu") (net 3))
 (segment (start 135.033189 92.233189) (end 135.561068 92.761068) (width 0.2) (layer "F.Cu") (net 3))
 (segment (start 131.41686 92.233189) (end 135.033189 92.233189) (width 0.2) (layer "F.Cu") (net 3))
 (segment (start 135.561068 92.761068) (end 135.561068 106.138932) (width 0.2) (layer "F.Cu") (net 3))
 (segment (start 111.35 113.45) (end 113.64 111.16) (width 0.2) (layer "F.Cu") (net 13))
 (segment (start 120.26 110.7) (end 120.72 111.16) (width 0.2) (layer "F.Cu") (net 13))
 (segment (start 113.64 111.16) (end 120.72 111.16) (width 0.2) (layer "F.Cu") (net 13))
 (segment (start 111.35 110.95) (end 112.75 110.95) (width 0.2) (layer "B.Cu") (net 17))
 (segment (start 114 112.2) (end 114 114.6) (width 0.2) (layer "B.Cu") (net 17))
 (segment (start 112.75 110.95) (end 114 112.2) (width 0.2) (layer "B.Cu") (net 17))
 (segment (start 114 114.6) (end 120.72 121.32) (width 0.2) (layer "B.Cu") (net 17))
 (segment (start 111.35 105.95) (end 112.97 105.95) (width 0.2) (layer "B.Cu") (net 14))
 (segment (start 112.97 105.95) (end 120.72 113.7) (width 0.2) (layer "B.Cu") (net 14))
 (segment (start 115.5 110.7) (end 115.5 113.56) (width 0.2) (layer "B.Cu") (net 16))
 (segment (start 115.5 113.56) (end 120.72 118.78) (width 0.2) (layer "B.Cu") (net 16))
 (segment (start 113.25 108.45) (end 115.5 110.7) (width 0.2) (layer "B.Cu") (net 16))
 (segment (start 111.35 108.45) (end 113.25 108.45) (width 0.2) (layer "B.Cu") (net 16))
 (segment (start 111.35 118.45) (end 113.56 116.24) (width 0.2) (layer "F.Cu") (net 15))
 (segment (start 113.56 116.24) (end 120.72 116.24) (width 0.2) (layer "F.Cu") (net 15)))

